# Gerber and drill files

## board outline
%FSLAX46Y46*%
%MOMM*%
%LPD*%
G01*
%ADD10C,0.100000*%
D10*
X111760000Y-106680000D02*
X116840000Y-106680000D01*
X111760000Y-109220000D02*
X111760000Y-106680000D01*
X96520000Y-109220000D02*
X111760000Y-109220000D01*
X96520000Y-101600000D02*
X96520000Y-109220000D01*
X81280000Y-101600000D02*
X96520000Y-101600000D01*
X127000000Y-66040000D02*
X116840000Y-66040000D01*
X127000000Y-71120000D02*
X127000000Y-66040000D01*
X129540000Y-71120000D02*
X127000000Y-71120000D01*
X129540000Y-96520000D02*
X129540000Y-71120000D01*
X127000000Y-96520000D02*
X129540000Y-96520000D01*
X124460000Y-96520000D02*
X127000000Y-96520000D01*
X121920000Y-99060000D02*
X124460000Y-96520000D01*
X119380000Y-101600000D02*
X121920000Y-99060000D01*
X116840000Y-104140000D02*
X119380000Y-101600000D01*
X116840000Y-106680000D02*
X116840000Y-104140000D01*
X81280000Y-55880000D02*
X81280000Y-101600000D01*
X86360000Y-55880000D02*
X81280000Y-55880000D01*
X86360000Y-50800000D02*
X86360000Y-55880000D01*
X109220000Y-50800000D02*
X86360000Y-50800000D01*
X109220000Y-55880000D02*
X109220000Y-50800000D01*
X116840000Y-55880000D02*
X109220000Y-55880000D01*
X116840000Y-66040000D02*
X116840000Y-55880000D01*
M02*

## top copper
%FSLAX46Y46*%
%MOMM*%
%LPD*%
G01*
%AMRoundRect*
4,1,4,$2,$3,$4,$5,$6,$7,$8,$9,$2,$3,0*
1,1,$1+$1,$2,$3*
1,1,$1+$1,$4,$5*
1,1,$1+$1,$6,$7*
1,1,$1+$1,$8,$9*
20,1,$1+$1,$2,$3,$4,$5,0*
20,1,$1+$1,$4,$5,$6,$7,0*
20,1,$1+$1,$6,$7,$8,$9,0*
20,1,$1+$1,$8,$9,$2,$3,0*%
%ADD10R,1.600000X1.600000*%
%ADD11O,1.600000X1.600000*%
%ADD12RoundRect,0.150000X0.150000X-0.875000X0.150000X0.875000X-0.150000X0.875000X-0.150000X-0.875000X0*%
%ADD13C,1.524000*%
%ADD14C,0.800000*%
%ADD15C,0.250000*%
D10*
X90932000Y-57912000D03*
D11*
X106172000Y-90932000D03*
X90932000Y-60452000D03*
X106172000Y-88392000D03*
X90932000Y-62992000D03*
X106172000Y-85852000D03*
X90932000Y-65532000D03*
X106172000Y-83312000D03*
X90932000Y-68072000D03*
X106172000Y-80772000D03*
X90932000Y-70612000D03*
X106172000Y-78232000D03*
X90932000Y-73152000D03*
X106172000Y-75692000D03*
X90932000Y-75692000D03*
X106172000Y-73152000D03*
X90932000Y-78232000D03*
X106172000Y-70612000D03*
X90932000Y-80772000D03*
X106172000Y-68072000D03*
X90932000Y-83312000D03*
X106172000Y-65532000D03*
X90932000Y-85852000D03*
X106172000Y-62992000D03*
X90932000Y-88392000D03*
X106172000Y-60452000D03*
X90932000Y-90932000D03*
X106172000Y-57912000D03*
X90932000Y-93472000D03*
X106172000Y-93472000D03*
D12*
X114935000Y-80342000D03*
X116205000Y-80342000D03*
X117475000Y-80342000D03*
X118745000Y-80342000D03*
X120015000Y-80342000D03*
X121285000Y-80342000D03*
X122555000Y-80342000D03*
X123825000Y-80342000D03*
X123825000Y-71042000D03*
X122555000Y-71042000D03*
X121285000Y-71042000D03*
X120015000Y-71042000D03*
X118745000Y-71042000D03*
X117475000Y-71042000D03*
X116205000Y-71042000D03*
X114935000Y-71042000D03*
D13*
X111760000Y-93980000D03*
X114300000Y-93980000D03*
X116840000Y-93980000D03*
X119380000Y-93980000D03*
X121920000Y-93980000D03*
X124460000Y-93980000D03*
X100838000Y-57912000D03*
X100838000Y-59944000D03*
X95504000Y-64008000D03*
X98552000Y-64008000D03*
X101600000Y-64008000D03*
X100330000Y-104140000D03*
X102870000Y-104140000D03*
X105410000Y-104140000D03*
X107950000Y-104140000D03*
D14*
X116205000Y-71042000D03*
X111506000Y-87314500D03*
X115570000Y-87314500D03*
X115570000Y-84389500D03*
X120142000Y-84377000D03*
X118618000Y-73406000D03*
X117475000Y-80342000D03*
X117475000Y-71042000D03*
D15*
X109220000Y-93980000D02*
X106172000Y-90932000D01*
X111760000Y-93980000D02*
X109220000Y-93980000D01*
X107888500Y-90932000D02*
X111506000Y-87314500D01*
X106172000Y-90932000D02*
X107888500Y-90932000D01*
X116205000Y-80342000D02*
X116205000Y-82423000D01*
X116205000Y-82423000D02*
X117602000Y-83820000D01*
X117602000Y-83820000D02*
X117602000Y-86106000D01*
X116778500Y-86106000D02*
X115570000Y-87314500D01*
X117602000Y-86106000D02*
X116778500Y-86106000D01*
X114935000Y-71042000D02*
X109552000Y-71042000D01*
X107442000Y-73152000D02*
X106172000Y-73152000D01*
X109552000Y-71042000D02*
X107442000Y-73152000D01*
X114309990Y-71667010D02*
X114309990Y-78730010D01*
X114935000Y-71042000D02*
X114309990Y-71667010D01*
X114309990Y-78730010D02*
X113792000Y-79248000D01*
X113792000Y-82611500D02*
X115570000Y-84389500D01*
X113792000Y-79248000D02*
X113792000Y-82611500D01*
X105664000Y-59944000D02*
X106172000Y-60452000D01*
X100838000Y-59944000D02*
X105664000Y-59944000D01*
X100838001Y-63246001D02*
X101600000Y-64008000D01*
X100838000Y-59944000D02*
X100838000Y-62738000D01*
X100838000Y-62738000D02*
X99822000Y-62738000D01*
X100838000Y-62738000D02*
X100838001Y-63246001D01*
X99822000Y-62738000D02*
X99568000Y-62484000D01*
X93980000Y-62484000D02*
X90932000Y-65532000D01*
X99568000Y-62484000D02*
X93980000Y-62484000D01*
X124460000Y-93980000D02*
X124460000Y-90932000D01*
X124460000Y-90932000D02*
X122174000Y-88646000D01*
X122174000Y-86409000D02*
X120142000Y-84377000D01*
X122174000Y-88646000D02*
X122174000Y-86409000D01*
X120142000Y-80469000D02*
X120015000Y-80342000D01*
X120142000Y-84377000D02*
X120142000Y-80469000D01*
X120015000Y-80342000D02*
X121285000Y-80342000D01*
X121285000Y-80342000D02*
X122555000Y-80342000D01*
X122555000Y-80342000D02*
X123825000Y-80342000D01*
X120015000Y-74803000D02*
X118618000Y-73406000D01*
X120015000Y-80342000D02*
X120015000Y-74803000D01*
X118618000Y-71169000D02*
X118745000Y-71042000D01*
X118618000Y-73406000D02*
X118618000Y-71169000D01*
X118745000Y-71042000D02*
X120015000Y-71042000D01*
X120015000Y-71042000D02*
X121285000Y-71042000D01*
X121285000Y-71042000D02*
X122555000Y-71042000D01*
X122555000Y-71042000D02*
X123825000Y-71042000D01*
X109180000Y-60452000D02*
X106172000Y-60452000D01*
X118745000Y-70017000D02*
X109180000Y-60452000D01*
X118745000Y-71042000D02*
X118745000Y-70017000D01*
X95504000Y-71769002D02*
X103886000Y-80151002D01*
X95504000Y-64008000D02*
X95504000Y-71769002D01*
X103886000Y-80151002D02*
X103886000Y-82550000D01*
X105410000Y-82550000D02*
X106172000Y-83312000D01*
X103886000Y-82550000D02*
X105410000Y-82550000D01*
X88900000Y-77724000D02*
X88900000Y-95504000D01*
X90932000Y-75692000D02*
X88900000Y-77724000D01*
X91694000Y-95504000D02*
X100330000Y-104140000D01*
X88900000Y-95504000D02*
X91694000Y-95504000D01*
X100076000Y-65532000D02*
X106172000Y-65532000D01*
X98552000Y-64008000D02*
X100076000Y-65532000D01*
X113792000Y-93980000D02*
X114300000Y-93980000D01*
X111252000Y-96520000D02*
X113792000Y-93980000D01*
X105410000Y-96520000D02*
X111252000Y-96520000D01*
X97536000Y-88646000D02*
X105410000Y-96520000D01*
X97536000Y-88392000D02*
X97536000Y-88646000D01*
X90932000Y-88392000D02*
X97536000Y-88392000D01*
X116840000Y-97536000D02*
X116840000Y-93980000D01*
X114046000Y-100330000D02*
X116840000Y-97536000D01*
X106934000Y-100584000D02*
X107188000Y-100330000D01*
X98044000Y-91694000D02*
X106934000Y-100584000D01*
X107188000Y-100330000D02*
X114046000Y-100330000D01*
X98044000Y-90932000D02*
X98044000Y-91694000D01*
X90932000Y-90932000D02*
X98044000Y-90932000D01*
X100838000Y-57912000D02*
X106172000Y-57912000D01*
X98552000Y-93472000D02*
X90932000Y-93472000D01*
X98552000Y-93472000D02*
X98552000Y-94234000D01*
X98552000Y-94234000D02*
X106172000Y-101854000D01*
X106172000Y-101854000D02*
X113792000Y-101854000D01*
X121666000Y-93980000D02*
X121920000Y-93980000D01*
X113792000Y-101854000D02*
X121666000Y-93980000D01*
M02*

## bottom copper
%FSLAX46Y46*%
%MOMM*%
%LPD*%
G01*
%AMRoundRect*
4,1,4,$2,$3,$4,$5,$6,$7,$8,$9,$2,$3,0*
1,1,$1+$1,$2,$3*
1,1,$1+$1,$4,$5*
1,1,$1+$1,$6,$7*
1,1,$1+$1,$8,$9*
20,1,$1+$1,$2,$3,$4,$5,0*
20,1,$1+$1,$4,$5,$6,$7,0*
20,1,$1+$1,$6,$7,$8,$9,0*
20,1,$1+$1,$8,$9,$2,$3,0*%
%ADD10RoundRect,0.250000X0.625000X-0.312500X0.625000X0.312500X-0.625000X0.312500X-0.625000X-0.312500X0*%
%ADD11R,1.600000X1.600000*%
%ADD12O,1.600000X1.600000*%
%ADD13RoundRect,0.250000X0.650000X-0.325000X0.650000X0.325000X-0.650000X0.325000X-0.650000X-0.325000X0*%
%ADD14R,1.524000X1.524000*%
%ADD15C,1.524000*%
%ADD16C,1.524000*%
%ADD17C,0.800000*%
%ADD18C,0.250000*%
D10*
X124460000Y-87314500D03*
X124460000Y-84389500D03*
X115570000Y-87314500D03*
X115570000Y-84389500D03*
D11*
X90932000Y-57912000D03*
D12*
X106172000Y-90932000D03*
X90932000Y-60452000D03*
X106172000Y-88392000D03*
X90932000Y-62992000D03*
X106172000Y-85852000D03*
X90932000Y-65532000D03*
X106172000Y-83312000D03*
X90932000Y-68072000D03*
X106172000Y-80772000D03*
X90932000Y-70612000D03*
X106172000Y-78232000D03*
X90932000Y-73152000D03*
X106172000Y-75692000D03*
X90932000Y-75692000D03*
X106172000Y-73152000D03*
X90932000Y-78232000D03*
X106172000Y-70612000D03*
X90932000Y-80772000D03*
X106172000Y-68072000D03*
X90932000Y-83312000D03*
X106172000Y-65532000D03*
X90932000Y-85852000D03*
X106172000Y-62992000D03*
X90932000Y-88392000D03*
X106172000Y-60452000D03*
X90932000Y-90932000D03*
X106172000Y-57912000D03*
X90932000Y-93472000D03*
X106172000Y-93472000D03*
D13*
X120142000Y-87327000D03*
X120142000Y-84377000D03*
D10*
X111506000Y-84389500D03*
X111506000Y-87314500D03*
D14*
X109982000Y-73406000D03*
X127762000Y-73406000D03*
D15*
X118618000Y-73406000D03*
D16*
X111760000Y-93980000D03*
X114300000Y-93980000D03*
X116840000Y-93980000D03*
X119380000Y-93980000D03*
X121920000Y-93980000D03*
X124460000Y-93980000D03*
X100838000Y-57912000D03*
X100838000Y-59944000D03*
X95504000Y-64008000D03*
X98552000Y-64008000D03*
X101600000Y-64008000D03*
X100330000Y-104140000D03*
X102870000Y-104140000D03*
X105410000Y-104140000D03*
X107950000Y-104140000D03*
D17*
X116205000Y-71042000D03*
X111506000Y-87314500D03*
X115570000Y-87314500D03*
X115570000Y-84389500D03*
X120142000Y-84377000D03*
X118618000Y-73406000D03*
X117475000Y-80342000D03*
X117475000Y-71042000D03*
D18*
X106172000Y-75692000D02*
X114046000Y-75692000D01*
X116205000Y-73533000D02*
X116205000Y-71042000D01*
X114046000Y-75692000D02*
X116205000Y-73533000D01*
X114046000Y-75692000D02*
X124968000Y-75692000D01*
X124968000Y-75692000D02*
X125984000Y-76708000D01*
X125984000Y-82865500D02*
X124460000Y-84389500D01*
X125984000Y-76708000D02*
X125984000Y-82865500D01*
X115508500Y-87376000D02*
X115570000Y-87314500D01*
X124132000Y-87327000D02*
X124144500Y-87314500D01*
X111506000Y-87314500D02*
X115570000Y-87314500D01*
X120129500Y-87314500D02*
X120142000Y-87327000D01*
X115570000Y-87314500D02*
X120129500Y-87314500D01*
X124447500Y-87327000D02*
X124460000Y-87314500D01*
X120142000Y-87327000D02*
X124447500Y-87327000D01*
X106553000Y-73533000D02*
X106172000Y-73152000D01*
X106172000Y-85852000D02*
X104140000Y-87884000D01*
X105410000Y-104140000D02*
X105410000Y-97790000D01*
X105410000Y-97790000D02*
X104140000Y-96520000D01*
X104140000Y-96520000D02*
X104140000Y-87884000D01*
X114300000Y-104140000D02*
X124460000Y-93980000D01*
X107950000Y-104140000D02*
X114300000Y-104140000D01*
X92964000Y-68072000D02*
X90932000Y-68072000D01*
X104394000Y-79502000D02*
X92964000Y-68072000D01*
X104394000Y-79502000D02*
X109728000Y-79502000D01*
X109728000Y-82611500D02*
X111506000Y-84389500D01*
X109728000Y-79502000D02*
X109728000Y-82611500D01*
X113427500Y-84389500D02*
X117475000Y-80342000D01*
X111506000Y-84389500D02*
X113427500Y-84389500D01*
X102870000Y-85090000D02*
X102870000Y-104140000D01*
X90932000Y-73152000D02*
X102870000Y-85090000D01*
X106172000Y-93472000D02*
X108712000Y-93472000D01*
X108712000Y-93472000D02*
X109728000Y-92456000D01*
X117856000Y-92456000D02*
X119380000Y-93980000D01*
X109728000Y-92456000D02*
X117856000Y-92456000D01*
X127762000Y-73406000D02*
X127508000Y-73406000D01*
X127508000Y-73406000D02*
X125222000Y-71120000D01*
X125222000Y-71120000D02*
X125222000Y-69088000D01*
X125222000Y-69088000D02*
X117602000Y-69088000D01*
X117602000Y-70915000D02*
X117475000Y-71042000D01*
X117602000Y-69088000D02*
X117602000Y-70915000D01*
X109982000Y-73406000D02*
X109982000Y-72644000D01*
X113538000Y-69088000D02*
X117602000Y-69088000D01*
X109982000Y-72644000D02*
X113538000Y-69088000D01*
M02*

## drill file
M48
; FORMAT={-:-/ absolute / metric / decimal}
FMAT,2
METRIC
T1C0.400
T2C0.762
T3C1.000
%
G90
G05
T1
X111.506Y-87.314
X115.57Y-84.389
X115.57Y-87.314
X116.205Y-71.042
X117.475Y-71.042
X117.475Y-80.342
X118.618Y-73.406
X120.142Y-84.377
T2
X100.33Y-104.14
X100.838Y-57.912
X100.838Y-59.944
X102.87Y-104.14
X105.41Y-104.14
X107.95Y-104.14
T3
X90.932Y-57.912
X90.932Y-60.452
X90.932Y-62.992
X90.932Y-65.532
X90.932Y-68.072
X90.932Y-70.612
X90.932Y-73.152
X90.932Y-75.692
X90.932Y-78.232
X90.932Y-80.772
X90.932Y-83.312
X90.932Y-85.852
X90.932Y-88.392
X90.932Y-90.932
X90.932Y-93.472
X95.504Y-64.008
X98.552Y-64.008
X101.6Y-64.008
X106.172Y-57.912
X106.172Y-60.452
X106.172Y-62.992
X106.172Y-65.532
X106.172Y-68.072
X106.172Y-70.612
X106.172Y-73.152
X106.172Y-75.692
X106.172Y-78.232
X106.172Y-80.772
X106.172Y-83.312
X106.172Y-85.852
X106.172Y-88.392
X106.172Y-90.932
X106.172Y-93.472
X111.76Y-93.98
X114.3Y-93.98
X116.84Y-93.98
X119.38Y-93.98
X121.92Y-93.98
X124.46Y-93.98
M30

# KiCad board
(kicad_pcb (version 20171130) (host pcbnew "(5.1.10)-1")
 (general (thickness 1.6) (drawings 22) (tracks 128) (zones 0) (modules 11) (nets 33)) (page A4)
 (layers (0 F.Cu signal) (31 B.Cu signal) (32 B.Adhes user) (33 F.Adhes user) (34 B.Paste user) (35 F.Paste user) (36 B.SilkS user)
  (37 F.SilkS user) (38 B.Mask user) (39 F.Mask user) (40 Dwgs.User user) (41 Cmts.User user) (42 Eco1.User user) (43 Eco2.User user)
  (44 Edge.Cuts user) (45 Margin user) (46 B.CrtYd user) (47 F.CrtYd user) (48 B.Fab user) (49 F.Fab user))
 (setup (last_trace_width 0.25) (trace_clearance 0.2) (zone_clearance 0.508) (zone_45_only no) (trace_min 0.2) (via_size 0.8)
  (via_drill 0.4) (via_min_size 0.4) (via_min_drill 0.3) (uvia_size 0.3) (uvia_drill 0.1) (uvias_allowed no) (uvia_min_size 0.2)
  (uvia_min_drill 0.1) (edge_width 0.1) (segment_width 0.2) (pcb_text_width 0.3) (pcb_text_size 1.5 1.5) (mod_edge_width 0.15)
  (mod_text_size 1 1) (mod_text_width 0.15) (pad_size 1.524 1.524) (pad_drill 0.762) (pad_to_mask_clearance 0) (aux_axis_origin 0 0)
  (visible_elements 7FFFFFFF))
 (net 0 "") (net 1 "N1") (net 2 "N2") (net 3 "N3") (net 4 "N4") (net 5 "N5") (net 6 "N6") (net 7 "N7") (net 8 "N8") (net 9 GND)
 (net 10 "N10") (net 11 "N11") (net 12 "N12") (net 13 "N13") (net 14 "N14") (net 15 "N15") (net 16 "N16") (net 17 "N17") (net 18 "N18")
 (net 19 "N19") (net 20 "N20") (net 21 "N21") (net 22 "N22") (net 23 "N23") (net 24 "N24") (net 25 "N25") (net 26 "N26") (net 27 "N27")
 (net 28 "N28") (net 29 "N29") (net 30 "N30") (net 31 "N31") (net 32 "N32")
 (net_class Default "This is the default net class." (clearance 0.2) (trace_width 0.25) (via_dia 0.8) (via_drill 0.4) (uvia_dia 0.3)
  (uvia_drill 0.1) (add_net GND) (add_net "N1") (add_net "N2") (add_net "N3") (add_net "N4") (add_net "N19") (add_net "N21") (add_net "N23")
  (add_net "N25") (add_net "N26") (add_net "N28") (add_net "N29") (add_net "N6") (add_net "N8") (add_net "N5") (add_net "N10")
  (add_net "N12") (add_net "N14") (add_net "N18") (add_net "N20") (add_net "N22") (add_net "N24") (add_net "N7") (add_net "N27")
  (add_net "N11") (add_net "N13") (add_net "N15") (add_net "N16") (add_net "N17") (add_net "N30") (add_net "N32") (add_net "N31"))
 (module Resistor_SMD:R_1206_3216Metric (layer B.Cu) (at 124.46 85.852 90)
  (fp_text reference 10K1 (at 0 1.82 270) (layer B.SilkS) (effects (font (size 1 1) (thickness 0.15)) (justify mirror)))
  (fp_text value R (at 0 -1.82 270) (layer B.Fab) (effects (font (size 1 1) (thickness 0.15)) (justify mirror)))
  (pad 1 smd roundrect (at -1.4625 0 90) (size 1.125 1.75) (layers B.Cu B.Paste B.Mask) (roundrect_rratio 0.222222) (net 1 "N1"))
  (pad 2 smd roundrect (at 1.4625 0 90) (size 1.125 1.75) (layers B.Cu B.Paste B.Mask) (roundrect_rratio 0.222222) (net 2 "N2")))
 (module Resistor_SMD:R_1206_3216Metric (layer B.Cu) (at 115.57 85.852 90)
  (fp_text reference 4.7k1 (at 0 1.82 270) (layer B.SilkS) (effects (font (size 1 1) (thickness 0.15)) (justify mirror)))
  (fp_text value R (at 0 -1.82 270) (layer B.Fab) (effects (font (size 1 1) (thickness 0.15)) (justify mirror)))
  (pad 1 smd roundrect (at -1.4625 0 90) (size 1.125 1.75) (layers B.Cu B.Paste B.Mask) (roundrect_rratio 0.222222) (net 1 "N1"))
  (pad 2 smd roundrect (at 1.4625 0 90) (size 1.125 1.75) (layers B.Cu B.Paste B.Mask) (roundrect_rratio 0.222222) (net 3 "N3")))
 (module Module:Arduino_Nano (layer F.Cu) (at 90.932 57.912)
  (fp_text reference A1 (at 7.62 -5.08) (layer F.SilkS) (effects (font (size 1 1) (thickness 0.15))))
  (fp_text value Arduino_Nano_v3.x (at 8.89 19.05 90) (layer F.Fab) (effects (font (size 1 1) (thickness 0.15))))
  (pad 1 thru_hole rect (at 0 0) (size 1.6 1.6) (drill 1) (layers *.Cu *.Mask) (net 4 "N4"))
  (pad 17 thru_hole oval (at 15.24 33.02) (size 1.6 1.6) (drill 1) (layers *.Cu *.Mask) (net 1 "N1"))
  (pad 2 thru_hole oval (at 0 2.54) (size 1.6 1.6) (drill 1) (layers *.Cu *.Mask) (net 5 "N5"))
  (pad 18 thru_hole oval (at 15.24 30.48) (size 1.6 1.6) (drill 1) (layers *.Cu *.Mask) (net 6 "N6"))
  (pad 3 thru_hole oval (at 0 5.08) (size 1.6 1.6) (drill 1) (layers *.Cu *.Mask) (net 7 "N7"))
  (pad 19 thru_hole oval (at 15.24 27.94) (size 1.6 1.6) (drill 1) (layers *.Cu *.Mask) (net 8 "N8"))
  (pad 4 thru_hole oval (at 0 7.62) (size 1.6 1.6) (drill 1) (layers *.Cu *.Mask) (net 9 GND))
  (pad 20 thru_hole oval (at 15.24 25.4) (size 1.6 1.6) (drill 1) (layers *.Cu *.Mask) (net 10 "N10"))
  (pad 5 thru_hole oval (at 0 10.16) (size 1.6 1.6) (drill 1) (layers *.Cu *.Mask) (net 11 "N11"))
  (pad 21 thru_hole oval (at 15.24 22.86) (size 1.6 1.6) (drill 1) (layers *.Cu *.Mask) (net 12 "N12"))
  (pad 6 thru_hole oval (at 0 12.7) (size 1.6 1.6) (drill 1) (layers *.Cu *.Mask) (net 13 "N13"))
  (pad 22 thru_hole oval (at 15.24 20.32) (size 1.6 1.6) (drill 1) (layers *.Cu *.Mask) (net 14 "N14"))
  (pad 7 thru_hole oval (at 0 15.24) (size 1.6 1.6) (drill 1) (layers *.Cu *.Mask) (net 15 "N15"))
  (pad 23 thru_hole oval (at 15.24 17.78) (size 1.6 1.6) (drill 1) (layers *.Cu *.Mask) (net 2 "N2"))
  (pad 8 thru_hole oval (at 0 17.78) (size 1.6 1.6) (drill 1) (layers *.Cu *.Mask) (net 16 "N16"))
  (pad 24 thru_hole oval (at 15.24 15.24) (size 1.6 1.6) (drill 1) (layers *.Cu *.Mask) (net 3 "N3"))
  (pad 9 thru_hole oval (at 0 20.32) (size 1.6 1.6) (drill 1) (layers *.Cu *.Mask) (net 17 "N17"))
  (pad 25 thru_hole oval (at 15.24 12.7) (size 1.6 1.6) (drill 1) (layers *.Cu *.Mask) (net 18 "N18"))
  (pad 10 thru_hole oval (at 0 22.86) (size 1.6 1.6) (drill 1) (layers *.Cu *.Mask) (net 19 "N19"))
  (pad 26 thru_hole oval (at 15.24 10.16) (size 1.6 1.6) (drill 1) (layers *.Cu *.Mask) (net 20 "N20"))
  (pad 11 thru_hole oval (at 0 25.4) (size 1.6 1.6) (drill 1) (layers *.Cu *.Mask) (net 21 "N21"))
  (pad 27 thru_hole oval (at 15.24 7.62) (size 1.6 1.6) (drill 1) (layers *.Cu *.Mask) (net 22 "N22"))
  (pad 12 thru_hole oval (at 0 27.94) (size 1.6 1.6) (drill 1) (layers *.Cu *.Mask) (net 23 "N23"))
  (pad 28 thru_hole oval (at 15.24 5.08) (size 1.6 1.6) (drill 1) (layers *.Cu *.Mask) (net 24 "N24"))
  (pad 13 thru_hole oval (at 0 30.48) (size 1.6 1.6) (drill 1) (layers *.Cu *.Mask) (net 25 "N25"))
  (pad 29 thru_hole oval (at 15.24 2.54) (size 1.6 1.6) (drill 1) (layers *.Cu *.Mask) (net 9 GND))
  (pad 14 thru_hole oval (at 0 33.02) (size 1.6 1.6) (drill 1) (layers *.Cu *.Mask) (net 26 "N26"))
  (pad 30 thru_hole oval (at 15.24 0) (size 1.6 1.6) (drill 1) (layers *.Cu *.Mask) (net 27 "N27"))
  (pad 15 thru_hole oval (at 0 35.56) (size 1.6 1.6) (drill 1) (layers *.Cu *.Mask) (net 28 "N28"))
  (pad 16 thru_hole oval (at 15.24 35.56) (size 1.6 1.6) (drill 1) (layers *.Cu *.Mask) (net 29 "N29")))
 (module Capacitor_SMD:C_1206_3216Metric (layer B.Cu) (at 120.142 85.852 90)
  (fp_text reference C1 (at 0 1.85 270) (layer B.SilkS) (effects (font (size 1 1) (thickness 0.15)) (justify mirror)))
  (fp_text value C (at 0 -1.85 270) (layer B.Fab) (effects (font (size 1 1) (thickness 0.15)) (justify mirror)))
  (pad 1 smd roundrect (at -1.475 0 90) (size 1.15 1.8) (layers B.Cu B.Paste B.Mask) (roundrect_rratio 0.217391) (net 1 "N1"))
  (pad 2 smd roundrect (at 1.475 0 90) (size 1.15 1.8) (layers B.Cu B.Paste B.Mask) (roundrect_rratio 0.217391) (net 9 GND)))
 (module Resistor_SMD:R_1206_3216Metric (layer B.Cu) (at 111.506 85.852 90)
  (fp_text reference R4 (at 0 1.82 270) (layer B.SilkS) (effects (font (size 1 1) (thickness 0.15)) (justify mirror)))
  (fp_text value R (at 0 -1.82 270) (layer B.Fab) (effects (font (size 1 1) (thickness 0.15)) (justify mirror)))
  (pad 2 smd roundrect (at 1.4625 0 90) (size 1.125 1.75) (layers B.Cu B.Paste B.Mask) (roundrect_rratio 0.222222) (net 11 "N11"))
  (pad 1 smd roundrect (at -1.4625 0 90) (size 1.125 1.75) (layers B.Cu B.Paste B.Mask) (roundrect_rratio 0.222222) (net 1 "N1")))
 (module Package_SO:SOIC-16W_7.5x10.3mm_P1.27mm (layer F.Cu) (at 119.38 75.692 90)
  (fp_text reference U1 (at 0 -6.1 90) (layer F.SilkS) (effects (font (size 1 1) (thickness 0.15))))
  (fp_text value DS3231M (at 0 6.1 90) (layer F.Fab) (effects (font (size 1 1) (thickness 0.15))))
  (pad 1 smd roundrect (at -4.65 -4.445 90) (size 2.05 0.6) (layers F.Cu F.Paste F.Mask) (roundrect_rratio 0.25) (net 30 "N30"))
  (pad 2 smd roundrect (at -4.65 -3.175 90) (size 2.05 0.6) (layers F.Cu F.Paste F.Mask) (roundrect_rratio 0.25) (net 1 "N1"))
  (pad 3 smd roundrect (at -4.65 -1.905 90) (size 2.05 0.6) (layers F.Cu F.Paste F.Mask) (roundrect_rratio 0.25) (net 11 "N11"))
  (pad 4 smd roundrect (at -4.65 -0.635 90) (size 2.05 0.6) (layers F.Cu F.Paste F.Mask) (roundrect_rratio 0.25) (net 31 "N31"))
  (pad 5 smd roundrect (at -4.65 0.635 90) (size 2.05 0.6) (layers F.Cu F.Paste F.Mask) (roundrect_rratio 0.25) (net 9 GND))
  (pad 6 smd roundrect (at -4.65 1.905 90) (size 2.05 0.6) (layers F.Cu F.Paste F.Mask) (roundrect_rratio 0.25) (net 9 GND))
  (pad 7 smd roundrect (at -4.65 3.175 90) (size 2.05 0.6) (layers F.Cu F.Paste F.Mask) (roundrect_rratio 0.25) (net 9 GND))
  (pad 8 smd roundrect (at -4.65 4.445 90) (size 2.05 0.6) (layers F.Cu F.Paste F.Mask) (roundrect_rratio 0.25) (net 9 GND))
  (pad 9 smd roundrect (at 4.65 4.445 90) (size 2.05 0.6) (layers F.Cu F.Paste F.Mask) (roundrect_rratio 0.25) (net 9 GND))
  (pad 10 smd roundrect (at 4.65 3.175 90) (size 2.05 0.6) (layers F.Cu F.Paste F.Mask) (roundrect_rratio 0.25) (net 9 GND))
  (pad 11 smd roundrect (at 4.65 1.905 90) (size 2.05 0.6) (layers F.Cu F.Paste F.Mask) (roundrect_rratio 0.25) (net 9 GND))
  (pad 12 smd roundrect (at 4.65 0.635 90) (size 2.05 0.6) (layers F.Cu F.Paste F.Mask) (roundrect_rratio 0.25) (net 9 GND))
  (pad 13 smd roundrect (at 4.65 -0.635 90) (size 2.05 0.6) (layers F.Cu F.Paste F.Mask) (roundrect_rratio 0.25) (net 9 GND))
  (pad 14 smd roundrect (at 4.65 -1.905 90) (size 2.05 0.6) (layers F.Cu F.Paste F.Mask) (roundrect_rratio 0.25) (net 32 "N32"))
  (pad 15 smd roundrect (at 4.65 -3.175 90) (size 2.05 0.6) (layers F.Cu F.Paste F.Mask) (roundrect_rratio 0.25) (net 2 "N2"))
  (pad 16 smd roundrect (at 4.65 -4.445 90) (size 2.05 0.6) (layers F.Cu F.Paste F.Mask) (roundrect_rratio 0.25) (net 3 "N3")))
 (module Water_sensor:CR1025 (layer B.Cu) (at 125.222 73.406 270)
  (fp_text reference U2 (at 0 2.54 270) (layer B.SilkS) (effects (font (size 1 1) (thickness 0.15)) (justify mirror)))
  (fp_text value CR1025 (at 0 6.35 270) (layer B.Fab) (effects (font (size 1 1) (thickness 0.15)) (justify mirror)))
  (pad 1 smd rect (at 0 15.24 270) (size 1.524 1.524) (layers B.Cu B.Paste B.Mask) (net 32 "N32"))
  (pad 2 smd rect (at 0 -2.54 270) (size 1.524 1.524) (layers B.Cu B.Paste B.Mask) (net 32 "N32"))
  (pad 3 smd circle (at 0 6.604 270) (size 1.524 1.524) (layers B.Cu B.Paste B.Mask) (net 9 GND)))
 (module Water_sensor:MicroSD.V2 (layer F.Cu) (at 119.38 91.44)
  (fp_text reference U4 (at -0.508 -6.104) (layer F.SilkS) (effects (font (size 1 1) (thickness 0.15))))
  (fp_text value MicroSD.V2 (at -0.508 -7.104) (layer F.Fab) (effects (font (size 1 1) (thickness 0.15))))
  (pad 1 thru_hole circle (at -7.62 2.54) (size 1.524 1.524) (drill 1) (layers *.Cu *.Mask) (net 1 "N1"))
  (pad 2 thru_hole circle (at -5.08 2.54) (size 1.524 1.524) (drill 1) (layers *.Cu *.Mask) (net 25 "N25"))
  (pad 3 thru_hole circle (at -2.54 2.54) (size 1.524 1.524) (drill 1) (layers *.Cu *.Mask) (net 26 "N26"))
  (pad 4 thru_hole circle (at 0 2.54) (size 1.524 1.524) (drill 1) (layers *.Cu *.Mask) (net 29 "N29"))
  (pad 5 thru_hole circle (at 2.54 2.54) (size 1.524 1.524) (drill 1) (layers *.Cu *.Mask) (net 28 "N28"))
  (pad 6 thru_hole circle (at 5.08 2.54) (size 1.524 1.524) (drill 1) (layers *.Cu *.Mask) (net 9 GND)))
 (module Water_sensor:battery (layer F.Cu) (at 102.87 58.928 270)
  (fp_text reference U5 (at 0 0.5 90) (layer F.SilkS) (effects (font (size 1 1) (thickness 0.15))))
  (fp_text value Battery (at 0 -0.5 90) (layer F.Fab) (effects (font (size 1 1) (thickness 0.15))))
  (pad 1 thru_hole circle (at -1.016 2.032 270) (size 1.524 1.524) (drill 0.762) (layers *.Cu *.Mask) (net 27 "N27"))
  (pad 2 thru_hole circle (at 1.016 2.032 270) (size 1.524 1.524) (drill 0.762) (layers *.Cu *.Mask) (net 9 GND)))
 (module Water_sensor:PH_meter (layer B.Cu) (at 98.552 62.992)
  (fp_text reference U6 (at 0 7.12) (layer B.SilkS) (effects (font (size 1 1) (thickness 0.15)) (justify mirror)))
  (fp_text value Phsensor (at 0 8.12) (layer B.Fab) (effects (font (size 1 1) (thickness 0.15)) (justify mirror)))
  (pad 1 thru_hole circle (at -3.048 1.016) (size 1.524 1.524) (drill 1) (layers *.Cu *.Mask) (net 10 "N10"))
  (pad 2 thru_hole circle (at 0 1.016) (size 1.524 1.524) (drill 1) (layers *.Cu *.Mask) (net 22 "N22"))
  (pad 3 thru_hole circle (at 3.048 1.016) (size 1.524 1.524) (drill 1) (layers *.Cu *.Mask) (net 9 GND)))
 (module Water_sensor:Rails (layer F.Cu) (at 104.14 101.6)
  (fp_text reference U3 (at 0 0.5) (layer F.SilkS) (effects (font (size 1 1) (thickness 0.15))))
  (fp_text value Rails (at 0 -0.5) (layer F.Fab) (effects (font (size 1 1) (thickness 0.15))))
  (pad 1 thru_hole circle (at -3.81 2.54) (size 1.524 1.524) (drill 0.762) (layers *.Cu *.Mask) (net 16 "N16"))
  (pad 2 thru_hole circle (at -1.27 2.54) (size 1.524 1.524) (drill 0.762) (layers *.Cu *.Mask) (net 15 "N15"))
  (pad 3 thru_hole circle (at 1.27 2.54) (size 1.524 1.524) (drill 0.762) (layers *.Cu *.Mask) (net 8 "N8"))
  (pad 4 thru_hole circle (at 3.81 2.54) (size 1.524 1.524) (drill 0.762) (layers *.Cu *.Mask) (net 9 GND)))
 (gr_line (start 111.76 106.68) (end 116.84 106.68) (layer Edge.Cuts) (width 0.1))
 (gr_line (start 111.76 109.22) (end 111.76 106.68) (layer Edge.Cuts) (width 0.1))
 (gr_line (start 96.52 109.22) (end 111.76 109.22) (layer Edge.Cuts) (width 0.1))
 (gr_line (start 96.52 101.6) (end 96.52 109.22) (layer Edge.Cuts) (width 0.1))
 (gr_line (start 81.28 101.6) (end 96.52 101.6) (layer Edge.Cuts) (width 0.1))
 (gr_line (start 127 66.04) (end 116.84 66.04) (layer Edge.Cuts) (width 0.1))
 (gr_line (start 127 71.12) (end 127 66.04) (layer Edge.Cuts) (width 0.1))
 (gr_line (start 129.54 71.12) (end 127 71.12) (layer Edge.Cuts) (width 0.1))
 (gr_line (start 129.54 96.52) (end 129.54 71.12) (layer Edge.Cuts) (width 0.1))
 (gr_line (start 127 96.52) (end 129.54 96.52) (layer Edge.Cuts) (width 0.1))
 (gr_line (start 124.46 96.52) (end 127 96.52) (layer Edge.Cuts) (width 0.1))
 (gr_line (start 121.92 99.06) (end 124.46 96.52) (layer Edge.Cuts) (width 0.1))
 (gr_line (start 119.38 101.6) (end 121.92 99.06) (layer Edge.Cuts) (width 0.1))
 (gr_line (start 116.84 104.14) (end 119.38 101.6) (layer Edge.Cuts) (width 0.1))
 (gr_line (start 116.84 106.68) (end 116.84 104.14) (layer Edge.Cuts) (width 0.1))
 (gr_line (start 81.28 55.88) (end 81.28 101.6) (layer Edge.Cuts) (width 0.1))
 (gr_line (start 86.36 55.88) (end 81.28 55.88) (layer Edge.Cuts) (width 0.1))
 (gr_line (start 86.36 50.8) (end 86.36 55.88) (layer Edge.Cuts) (width 0.1))
 (gr_line (start 109.22 50.8) (end 86.36 50.8) (layer Edge.Cuts) (width 0.1))
 (gr_line (start 109.22 55.88) (end 109.22 50.8) (layer Edge.Cuts) (width 0.1))
 (gr_line (start 116.84 55.88) (end 109.22 55.88) (layer Edge.Cuts) (width 0.1))
 (gr_line (start 116.84 66.04) (end 116.84 55.88) (layer Edge.Cuts) (width 0.1))
 (segment (start 106.172 75.692) (end 114.046 75.692) (width 0.25) (layer B.Cu) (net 2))
 (via (at 116.205 71.042) (size 0.8) (drill 0.4) (layers F.Cu B.Cu) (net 2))
 (segment (start 116.205 73.533) (end 116.205 71.042) (width 0.25) (layer B.Cu) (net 2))
 (segment (start 114.046 75.692) (end 116.205 73.533) (width 0.25) (layer B.Cu) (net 2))
 (segment (start 114.046 75.692) (end 124.968 75.692) (width 0.25) (layer B.Cu) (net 2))
 (segment (start 124.968 75.692) (end 125.984 76.708) (width 0.25) (layer B.Cu) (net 2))
 (segment (start 125.984 82.8655) (end 124.46 84.3895) (width 0.25) (layer B.Cu) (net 2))
 (segment (start 125.984 76.708) (end 125.984 82.8655) (width 0.25) (layer B.Cu) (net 2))
 (segment (start 115.5085 87.376) (end 115.57 87.3145) (width 0.25) (layer B.Cu) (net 1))
 (segment (start 124.132 87.327) (end 124.1445 87.3145) (width 0.25) (layer B.Cu) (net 1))
 (segment (start 109.22 93.98) (end 106.172 90.932) (width 0.25) (layer F.Cu) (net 1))
 (segment (start 111.76 93.98) (end 109.22 93.98) (width 0.25) (layer F.Cu) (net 1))
 (via (at 111.506 87.3145) (size 0.8) (drill 0.4) (layers F.Cu B.Cu) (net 1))
 (segment (start 107.8885 90.932) (end 111.506 87.3145) (width 0.25) (layer F.Cu) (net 1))
 (segment (start 106.172 90.932) (end 107.8885 90.932) (width 0.25) (layer F.Cu) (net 1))
 (segment (start 111.506 87.3145) (end 115.57 87.3145) (width 0.25) (layer B.Cu) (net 1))
 (segment (start 120.1295 87.3145) (end 120.142 87.327) (width 0.25) (layer B.Cu) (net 1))
 (segment (start 115.57 87.3145) (end 120.1295 87.3145) (width 0.25) (layer B.Cu) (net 1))
 (segment (start 124.4475 87.327) (end 124.46 87.3145) (width 0.25) (layer B.Cu) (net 1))
 (segment (start 120.142 87.327) (end 124.4475 87.327) (width 0.25) (layer B.Cu) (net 1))
 (segment (start 116.205 80.342) (end 116.205 82.423) (width 0.25) (layer F.Cu) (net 1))
 (segment (start 116.205 82.423) (end 117.602 83.82) (width 0.25) (layer F.Cu) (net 1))
 (segment (start 117.602 83.82) (end 117.602 86.106) (width 0.25) (layer F.Cu) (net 1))
 (via (at 115.57 87.3145) (size 0.8) (drill 0.4) (layers F.Cu B.Cu) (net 1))
 (segment (start 116.7785 86.106) (end 115.57 87.3145) (width 0.25) (layer F.Cu) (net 1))
 (segment (start 117.602 86.106) (end 116.7785 86.106) (width 0.25) (layer F.Cu) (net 1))
 (segment (start 106.553 73.533) (end 106.172 73.152) (width 0.25) (layer B.Cu) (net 3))
 (segment (start 114.935 71.042) (end 109.552 71.042) (width 0.25) (layer F.Cu) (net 3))
 (segment (start 107.442 73.152) (end 106.172 73.152) (width 0.25) (layer F.Cu) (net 3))
 (segment (start 109.552 71.042) (end 107.442 73.152) (width 0.25) (layer F.Cu) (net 3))
 (segment (start 114.30999 71.66701) (end 114.30999 78.73001) (width 0.25) (layer F.Cu) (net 3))
 (segment (start 114.935 71.042) (end 114.30999 71.66701) (width 0.25) (layer F.Cu) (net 3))
 (segment (start 114.30999 78.73001) (end 113.792 79.248) (width 0.25) (layer F.Cu) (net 3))
 (via (at 115.57 84.3895) (size 0.8) (drill 0.4) (layers F.Cu B.Cu) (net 3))
 (segment (start 113.792 82.6115) (end 115.57 84.3895) (width 0.25) (layer F.Cu) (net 3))
 (segment (start 113.792 79.248) (end 113.792 82.6115) (width 0.25) (layer F.Cu) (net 3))
 (segment (start 106.172 85.852) (end 104.14 87.884) (width 0.25) (layer B.Cu) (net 8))
 (segment (start 105.41 104.14) (end 105.41 97.79) (width 0.25) (layer B.Cu) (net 8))
 (segment (start 105.41 97.79) (end 104.14 96.52) (width 0.25) (layer B.Cu) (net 8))
 (segment (start 104.14 96.52) (end 104.14 87.884) (width 0.25) (layer B.Cu) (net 8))
 (segment (start 105.664 59.944) (end 106.172 60.452) (width 0.25) (layer F.Cu) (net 9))
 (segment (start 100.838 59.944) (end 105.664 59.944) (width 0.25) (layer F.Cu) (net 9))
 (segment (start 100.838001 63.246001) (end 101.6 64.008) (width 0.25) (layer F.Cu) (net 9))
 (segment (start 100.838 59.944) (end 100.838 62.738) (width 0.25) (layer F.Cu) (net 9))
 (segment (start 100.838 62.738) (end 99.822 62.738) (width 0.25) (layer F.Cu) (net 9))
 (segment (start 100.838 62.738) (end 100.838001 63.246001) (width 0.25) (layer F.Cu) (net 9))
 (segment (start 99.822 62.738) (end 99.568 62.484) (width 0.25) (layer F.Cu) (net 9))
 (segment (start 93.98 62.484) (end 90.932 65.532) (width 0.25) (layer F.Cu) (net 9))
 (segment (start 99.568 62.484) (end 93.98 62.484) (width 0.25) (layer F.Cu) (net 9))
 (segment (start 124.46 93.98) (end 124.46 90.932) (width 0.25) (layer F.Cu) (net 9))
 (segment (start 124.46 90.932) (end 122.174 88.646) (width 0.25) (layer F.Cu) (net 9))
 (via (at 120.142 84.377) (size 0.8) (drill 0.4) (layers F.Cu B.Cu) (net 9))
 (segment (start 122.174 86.409) (end 120.142 84.377) (width 0.25) (layer F.Cu) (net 9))
 (segment (start 122.174 88.646) (end 122.174 86.409) (width 0.25) (layer F.Cu) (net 9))
 (segment (start 120.142 80.469) (end 120.015 80.342) (width 0.25) (layer F.Cu) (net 9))
 (segment (start 120.142 84.377) (end 120.142 80.469) (width 0.25) (layer F.Cu) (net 9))
 (segment (start 120.015 80.342) (end 121.285 80.342) (width 0.25) (layer F.Cu) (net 9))
 (segment (start 121.285 80.342) (end 122.555 80.342) (width 0.25) (layer F.Cu) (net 9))
 (segment (start 122.555 80.342) (end 123.825 80.342) (width 0.25) (layer F.Cu) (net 9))
 (via (at 118.618 73.406) (size 0.8) (drill 0.4) (layers F.Cu B.Cu) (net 9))
 (segment (start 120.015 74.803) (end 118.618 73.406) (width 0.25) (layer F.Cu) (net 9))
 (segment (start 120.015 80.342) (end 120.015 74.803) (width 0.25) (layer F.Cu) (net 9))
 (segment (start 118.618 71.169) (end 118.745 71.042) (width 0.25) (layer F.Cu) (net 9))
 (segment (start 118.618 73.406) (end 118.618 71.169) (width 0.25) (layer F.Cu) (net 9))
 (segment (start 118.745 71.042) (end 120.015 71.042) (width 0.25) (layer F.Cu) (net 9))
 (segment (start 120.015 71.042) (end 121.285 71.042) (width 0.25) (layer F.Cu) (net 9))
 (segment (start 121.285 71.042) (end 122.555 71.042) (width 0.25) (layer F.Cu) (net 9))
 (segment (start 122.555 71.042) (end 123.825 71.042) (width 0.25) (layer F.Cu) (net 9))
 (segment (start 109.18 60.452) (end 106.172 60.452) (width 0.25) (layer F.Cu) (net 9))
 (segment (start 118.745 70.017) (end 109.18 60.452) (width 0.25) (layer F.Cu) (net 9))
 (segment (start 118.745 71.042) (end 118.745 70.017) (width 0.25) (layer F.Cu) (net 9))
 (segment (start 114.3 104.14) (end 124.46 93.98) (width 0.25) (layer B.Cu) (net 9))
 (segment (start 107.95 104.14) (end 114.3 104.14) (width 0.25) (layer B.Cu) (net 9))
 (segment (start 95.504 71.769002) (end 103.886 80.151002) (width 0.25) (layer F.Cu) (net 10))
 (segment (start 95.504 64.008) (end 95.504 71.769002) (width 0.25) (layer F.Cu) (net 10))
 (segment (start 103.886 80.151002) (end 103.886 82.55) (width 0.25) (layer F.Cu) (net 10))
 (segment (start 105.41 82.55) (end 106.172 83.312) (width 0.25) (layer F.Cu) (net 10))
 (segment (start 103.886 82.55) (end 105.41 82.55) (width 0.25) (layer F.Cu) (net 10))
 (segment (start 92.964 68.072) (end 90.932 68.072) (width 0.25) (layer B.Cu) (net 11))
 (segment (start 104.394 79.502) (end 92.964 68.072) (width 0.25) (layer B.Cu) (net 11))
 (segment (start 104.394 79.502) (end 109.728 79.502) (width 0.25) (layer B.Cu) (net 11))
 (segment (start 109.728 82.6115) (end 111.506 84.3895) (width 0.25) (layer B.Cu) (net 11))
 (segment (start 109.728 79.502) (end 109.728 82.6115) (width 0.25) (layer B.Cu) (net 11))
 (via (at 117.475 80.342) (size 0.8) (drill 0.4) (layers F.Cu B.Cu) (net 11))
 (segment (start 113.4275 84.3895) (end 117.475 80.342) (width 0.25) (layer B.Cu) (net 11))
 (segment (start 111.506 84.3895) (end 113.4275 84.3895) (width 0.25) (layer B.Cu) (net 11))
 (segment (start 102.87 85.09) (end 102.87 104.14) (width 0.25) (layer B.Cu) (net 15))
 (segment (start 90.932 73.152) (end 102.87 85.09) (width 0.25) (layer B.Cu) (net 15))
 (segment (start 88.9 77.724) (end 88.9 95.504) (width 0.25) (layer F.Cu) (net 16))
 (segment (start 90.932 75.692) (end 88.9 77.724) (width 0.25) (layer F.Cu) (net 16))
 (segment (start 91.694 95.504) (end 100.33 104.14) (width 0.25) (layer F.Cu) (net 16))
 (segment (start 88.9 95.504) (end 91.694 95.504) (width 0.25) (layer F.Cu) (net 16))
 (segment (start 100.076 65.532) (end 106.172 65.532) (width 0.25) (layer F.Cu) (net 22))
 (segment (start 98.552 64.008) (end 100.076 65.532) (width 0.25) (layer F.Cu) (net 22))
 (segment (start 113.792 93.98) (end 114.3 93.98) (width 0.25) (layer F.Cu) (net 25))
 (segment (start 111.252 96.52) (end 113.792 93.98) (width 0.25) (layer F.Cu) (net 25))
 (segment (start 105.41 96.52) (end 111.252 96.52) (width 0.25) (layer F.Cu) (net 25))
 (segment (start 97.536 88.646) (end 105.41 96.52) (width 0.25) (layer F.Cu) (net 25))
 (segment (start 97.536 88.392) (end 97.536 88.646) (width 0.25) (layer F.Cu) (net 25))
 (segment (start 90.932 88.392) (end 97.536 88.392) (width 0.25) (layer F.Cu) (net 25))
 (segment (start 116.84 97.536) (end 116.84 93.98) (width 0.25) (layer F.Cu) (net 26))
 (segment (start 114.046 100.33) (end 116.84 97.536) (width 0.25) (layer F.Cu) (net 26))
 (segment (start 106.934 100.584) (end 107.188 100.33) (width 0.25) (layer F.Cu) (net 26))
 (segment (start 98.044 91.694) (end 106.934 100.584) (width 0.25) (layer F.Cu) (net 26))
 (segment (start 107.188 100.33) (end 114.046 100.33) (width 0.25) (layer F.Cu) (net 26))
 (segment (start 98.044 90.932) (end 98.044 91.694) (width 0.25) (layer F.Cu) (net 26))
 (segment (start 90.932 90.932) (end 98.044 90.932) (width 0.25) (layer F.Cu) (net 26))
 (segment (start 100.838 57.912) (end 106.172 57.912) (width 0.25) (layer F.Cu) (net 27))
 (segment (start 98.552 93.472) (end 90.932 93.472) (width 0.25) (layer F.Cu) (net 28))
 (segment (start 98.552 93.472) (end 98.552 94.234) (width 0.25) (layer F.Cu) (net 28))
 (segment (start 98.552 94.234) (end 106.172 101.854) (width 0.25) (layer F.Cu) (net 28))
 (segment (start 106.172 101.854) (end 113.792 101.854) (width 0.25) (layer F.Cu) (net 28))
 (segment (start 121.666 93.98) (end 121.92 93.98) (width 0.25) (layer F.Cu) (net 28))
 (segment (start 113.792 101.854) (end 121.666 93.98) (width 0.25) (layer F.Cu) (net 28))
 (segment (start 106.172 93.472) (end 108.712 93.472) (width 0.25) (layer B.Cu) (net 29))
 (segment (start 108.712 93.472) (end 109.728 92.456) (width 0.25) (layer B.Cu) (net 29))
 (segment (start 117.856 92.456) (end 119.38 93.98) (width 0.25) (layer B.Cu) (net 29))
 (segment (start 109.728 92.456) (end 117.856 92.456) (width 0.25) (layer B.Cu) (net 29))
 (segment (start 127.762 73.406) (end 127.508 73.406) (width 0.25) (layer B.Cu) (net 32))
 (segment (start 127.508 73.406) (end 125.222 71.12) (width 0.25) (layer B.Cu) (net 32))
 (segment (start 125.222 71.12) (end 125.222 69.088) (width 0.25) (layer B.Cu) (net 32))
 (segment (start 125.222 69.088) (end 117.602 69.088) (width 0.25) (layer B.Cu) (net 32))
 (segment (start 117.602 70.915) (end 117.475 71.042) (width 0.25) (layer B.Cu) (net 32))
 (via (at 117.475 71.042) (size 0.8) (drill 0.4) (layers F.Cu B.Cu) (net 32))
 (segment (start 117.602 69.088) (end 117.602 70.915) (width 0.25) (layer B.Cu) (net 32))
 (segment (start 109.982 73.406) (end 109.982 72.644) (width 0.25) (layer B.Cu) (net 32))
 (segment (start 113.538 69.088) (end 117.602 69.088) (width 0.25) (layer B.Cu) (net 32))
 (segment (start 109.982 72.644) (end 113.538 69.088) (width 0.25) (layer B.Cu) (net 32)))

